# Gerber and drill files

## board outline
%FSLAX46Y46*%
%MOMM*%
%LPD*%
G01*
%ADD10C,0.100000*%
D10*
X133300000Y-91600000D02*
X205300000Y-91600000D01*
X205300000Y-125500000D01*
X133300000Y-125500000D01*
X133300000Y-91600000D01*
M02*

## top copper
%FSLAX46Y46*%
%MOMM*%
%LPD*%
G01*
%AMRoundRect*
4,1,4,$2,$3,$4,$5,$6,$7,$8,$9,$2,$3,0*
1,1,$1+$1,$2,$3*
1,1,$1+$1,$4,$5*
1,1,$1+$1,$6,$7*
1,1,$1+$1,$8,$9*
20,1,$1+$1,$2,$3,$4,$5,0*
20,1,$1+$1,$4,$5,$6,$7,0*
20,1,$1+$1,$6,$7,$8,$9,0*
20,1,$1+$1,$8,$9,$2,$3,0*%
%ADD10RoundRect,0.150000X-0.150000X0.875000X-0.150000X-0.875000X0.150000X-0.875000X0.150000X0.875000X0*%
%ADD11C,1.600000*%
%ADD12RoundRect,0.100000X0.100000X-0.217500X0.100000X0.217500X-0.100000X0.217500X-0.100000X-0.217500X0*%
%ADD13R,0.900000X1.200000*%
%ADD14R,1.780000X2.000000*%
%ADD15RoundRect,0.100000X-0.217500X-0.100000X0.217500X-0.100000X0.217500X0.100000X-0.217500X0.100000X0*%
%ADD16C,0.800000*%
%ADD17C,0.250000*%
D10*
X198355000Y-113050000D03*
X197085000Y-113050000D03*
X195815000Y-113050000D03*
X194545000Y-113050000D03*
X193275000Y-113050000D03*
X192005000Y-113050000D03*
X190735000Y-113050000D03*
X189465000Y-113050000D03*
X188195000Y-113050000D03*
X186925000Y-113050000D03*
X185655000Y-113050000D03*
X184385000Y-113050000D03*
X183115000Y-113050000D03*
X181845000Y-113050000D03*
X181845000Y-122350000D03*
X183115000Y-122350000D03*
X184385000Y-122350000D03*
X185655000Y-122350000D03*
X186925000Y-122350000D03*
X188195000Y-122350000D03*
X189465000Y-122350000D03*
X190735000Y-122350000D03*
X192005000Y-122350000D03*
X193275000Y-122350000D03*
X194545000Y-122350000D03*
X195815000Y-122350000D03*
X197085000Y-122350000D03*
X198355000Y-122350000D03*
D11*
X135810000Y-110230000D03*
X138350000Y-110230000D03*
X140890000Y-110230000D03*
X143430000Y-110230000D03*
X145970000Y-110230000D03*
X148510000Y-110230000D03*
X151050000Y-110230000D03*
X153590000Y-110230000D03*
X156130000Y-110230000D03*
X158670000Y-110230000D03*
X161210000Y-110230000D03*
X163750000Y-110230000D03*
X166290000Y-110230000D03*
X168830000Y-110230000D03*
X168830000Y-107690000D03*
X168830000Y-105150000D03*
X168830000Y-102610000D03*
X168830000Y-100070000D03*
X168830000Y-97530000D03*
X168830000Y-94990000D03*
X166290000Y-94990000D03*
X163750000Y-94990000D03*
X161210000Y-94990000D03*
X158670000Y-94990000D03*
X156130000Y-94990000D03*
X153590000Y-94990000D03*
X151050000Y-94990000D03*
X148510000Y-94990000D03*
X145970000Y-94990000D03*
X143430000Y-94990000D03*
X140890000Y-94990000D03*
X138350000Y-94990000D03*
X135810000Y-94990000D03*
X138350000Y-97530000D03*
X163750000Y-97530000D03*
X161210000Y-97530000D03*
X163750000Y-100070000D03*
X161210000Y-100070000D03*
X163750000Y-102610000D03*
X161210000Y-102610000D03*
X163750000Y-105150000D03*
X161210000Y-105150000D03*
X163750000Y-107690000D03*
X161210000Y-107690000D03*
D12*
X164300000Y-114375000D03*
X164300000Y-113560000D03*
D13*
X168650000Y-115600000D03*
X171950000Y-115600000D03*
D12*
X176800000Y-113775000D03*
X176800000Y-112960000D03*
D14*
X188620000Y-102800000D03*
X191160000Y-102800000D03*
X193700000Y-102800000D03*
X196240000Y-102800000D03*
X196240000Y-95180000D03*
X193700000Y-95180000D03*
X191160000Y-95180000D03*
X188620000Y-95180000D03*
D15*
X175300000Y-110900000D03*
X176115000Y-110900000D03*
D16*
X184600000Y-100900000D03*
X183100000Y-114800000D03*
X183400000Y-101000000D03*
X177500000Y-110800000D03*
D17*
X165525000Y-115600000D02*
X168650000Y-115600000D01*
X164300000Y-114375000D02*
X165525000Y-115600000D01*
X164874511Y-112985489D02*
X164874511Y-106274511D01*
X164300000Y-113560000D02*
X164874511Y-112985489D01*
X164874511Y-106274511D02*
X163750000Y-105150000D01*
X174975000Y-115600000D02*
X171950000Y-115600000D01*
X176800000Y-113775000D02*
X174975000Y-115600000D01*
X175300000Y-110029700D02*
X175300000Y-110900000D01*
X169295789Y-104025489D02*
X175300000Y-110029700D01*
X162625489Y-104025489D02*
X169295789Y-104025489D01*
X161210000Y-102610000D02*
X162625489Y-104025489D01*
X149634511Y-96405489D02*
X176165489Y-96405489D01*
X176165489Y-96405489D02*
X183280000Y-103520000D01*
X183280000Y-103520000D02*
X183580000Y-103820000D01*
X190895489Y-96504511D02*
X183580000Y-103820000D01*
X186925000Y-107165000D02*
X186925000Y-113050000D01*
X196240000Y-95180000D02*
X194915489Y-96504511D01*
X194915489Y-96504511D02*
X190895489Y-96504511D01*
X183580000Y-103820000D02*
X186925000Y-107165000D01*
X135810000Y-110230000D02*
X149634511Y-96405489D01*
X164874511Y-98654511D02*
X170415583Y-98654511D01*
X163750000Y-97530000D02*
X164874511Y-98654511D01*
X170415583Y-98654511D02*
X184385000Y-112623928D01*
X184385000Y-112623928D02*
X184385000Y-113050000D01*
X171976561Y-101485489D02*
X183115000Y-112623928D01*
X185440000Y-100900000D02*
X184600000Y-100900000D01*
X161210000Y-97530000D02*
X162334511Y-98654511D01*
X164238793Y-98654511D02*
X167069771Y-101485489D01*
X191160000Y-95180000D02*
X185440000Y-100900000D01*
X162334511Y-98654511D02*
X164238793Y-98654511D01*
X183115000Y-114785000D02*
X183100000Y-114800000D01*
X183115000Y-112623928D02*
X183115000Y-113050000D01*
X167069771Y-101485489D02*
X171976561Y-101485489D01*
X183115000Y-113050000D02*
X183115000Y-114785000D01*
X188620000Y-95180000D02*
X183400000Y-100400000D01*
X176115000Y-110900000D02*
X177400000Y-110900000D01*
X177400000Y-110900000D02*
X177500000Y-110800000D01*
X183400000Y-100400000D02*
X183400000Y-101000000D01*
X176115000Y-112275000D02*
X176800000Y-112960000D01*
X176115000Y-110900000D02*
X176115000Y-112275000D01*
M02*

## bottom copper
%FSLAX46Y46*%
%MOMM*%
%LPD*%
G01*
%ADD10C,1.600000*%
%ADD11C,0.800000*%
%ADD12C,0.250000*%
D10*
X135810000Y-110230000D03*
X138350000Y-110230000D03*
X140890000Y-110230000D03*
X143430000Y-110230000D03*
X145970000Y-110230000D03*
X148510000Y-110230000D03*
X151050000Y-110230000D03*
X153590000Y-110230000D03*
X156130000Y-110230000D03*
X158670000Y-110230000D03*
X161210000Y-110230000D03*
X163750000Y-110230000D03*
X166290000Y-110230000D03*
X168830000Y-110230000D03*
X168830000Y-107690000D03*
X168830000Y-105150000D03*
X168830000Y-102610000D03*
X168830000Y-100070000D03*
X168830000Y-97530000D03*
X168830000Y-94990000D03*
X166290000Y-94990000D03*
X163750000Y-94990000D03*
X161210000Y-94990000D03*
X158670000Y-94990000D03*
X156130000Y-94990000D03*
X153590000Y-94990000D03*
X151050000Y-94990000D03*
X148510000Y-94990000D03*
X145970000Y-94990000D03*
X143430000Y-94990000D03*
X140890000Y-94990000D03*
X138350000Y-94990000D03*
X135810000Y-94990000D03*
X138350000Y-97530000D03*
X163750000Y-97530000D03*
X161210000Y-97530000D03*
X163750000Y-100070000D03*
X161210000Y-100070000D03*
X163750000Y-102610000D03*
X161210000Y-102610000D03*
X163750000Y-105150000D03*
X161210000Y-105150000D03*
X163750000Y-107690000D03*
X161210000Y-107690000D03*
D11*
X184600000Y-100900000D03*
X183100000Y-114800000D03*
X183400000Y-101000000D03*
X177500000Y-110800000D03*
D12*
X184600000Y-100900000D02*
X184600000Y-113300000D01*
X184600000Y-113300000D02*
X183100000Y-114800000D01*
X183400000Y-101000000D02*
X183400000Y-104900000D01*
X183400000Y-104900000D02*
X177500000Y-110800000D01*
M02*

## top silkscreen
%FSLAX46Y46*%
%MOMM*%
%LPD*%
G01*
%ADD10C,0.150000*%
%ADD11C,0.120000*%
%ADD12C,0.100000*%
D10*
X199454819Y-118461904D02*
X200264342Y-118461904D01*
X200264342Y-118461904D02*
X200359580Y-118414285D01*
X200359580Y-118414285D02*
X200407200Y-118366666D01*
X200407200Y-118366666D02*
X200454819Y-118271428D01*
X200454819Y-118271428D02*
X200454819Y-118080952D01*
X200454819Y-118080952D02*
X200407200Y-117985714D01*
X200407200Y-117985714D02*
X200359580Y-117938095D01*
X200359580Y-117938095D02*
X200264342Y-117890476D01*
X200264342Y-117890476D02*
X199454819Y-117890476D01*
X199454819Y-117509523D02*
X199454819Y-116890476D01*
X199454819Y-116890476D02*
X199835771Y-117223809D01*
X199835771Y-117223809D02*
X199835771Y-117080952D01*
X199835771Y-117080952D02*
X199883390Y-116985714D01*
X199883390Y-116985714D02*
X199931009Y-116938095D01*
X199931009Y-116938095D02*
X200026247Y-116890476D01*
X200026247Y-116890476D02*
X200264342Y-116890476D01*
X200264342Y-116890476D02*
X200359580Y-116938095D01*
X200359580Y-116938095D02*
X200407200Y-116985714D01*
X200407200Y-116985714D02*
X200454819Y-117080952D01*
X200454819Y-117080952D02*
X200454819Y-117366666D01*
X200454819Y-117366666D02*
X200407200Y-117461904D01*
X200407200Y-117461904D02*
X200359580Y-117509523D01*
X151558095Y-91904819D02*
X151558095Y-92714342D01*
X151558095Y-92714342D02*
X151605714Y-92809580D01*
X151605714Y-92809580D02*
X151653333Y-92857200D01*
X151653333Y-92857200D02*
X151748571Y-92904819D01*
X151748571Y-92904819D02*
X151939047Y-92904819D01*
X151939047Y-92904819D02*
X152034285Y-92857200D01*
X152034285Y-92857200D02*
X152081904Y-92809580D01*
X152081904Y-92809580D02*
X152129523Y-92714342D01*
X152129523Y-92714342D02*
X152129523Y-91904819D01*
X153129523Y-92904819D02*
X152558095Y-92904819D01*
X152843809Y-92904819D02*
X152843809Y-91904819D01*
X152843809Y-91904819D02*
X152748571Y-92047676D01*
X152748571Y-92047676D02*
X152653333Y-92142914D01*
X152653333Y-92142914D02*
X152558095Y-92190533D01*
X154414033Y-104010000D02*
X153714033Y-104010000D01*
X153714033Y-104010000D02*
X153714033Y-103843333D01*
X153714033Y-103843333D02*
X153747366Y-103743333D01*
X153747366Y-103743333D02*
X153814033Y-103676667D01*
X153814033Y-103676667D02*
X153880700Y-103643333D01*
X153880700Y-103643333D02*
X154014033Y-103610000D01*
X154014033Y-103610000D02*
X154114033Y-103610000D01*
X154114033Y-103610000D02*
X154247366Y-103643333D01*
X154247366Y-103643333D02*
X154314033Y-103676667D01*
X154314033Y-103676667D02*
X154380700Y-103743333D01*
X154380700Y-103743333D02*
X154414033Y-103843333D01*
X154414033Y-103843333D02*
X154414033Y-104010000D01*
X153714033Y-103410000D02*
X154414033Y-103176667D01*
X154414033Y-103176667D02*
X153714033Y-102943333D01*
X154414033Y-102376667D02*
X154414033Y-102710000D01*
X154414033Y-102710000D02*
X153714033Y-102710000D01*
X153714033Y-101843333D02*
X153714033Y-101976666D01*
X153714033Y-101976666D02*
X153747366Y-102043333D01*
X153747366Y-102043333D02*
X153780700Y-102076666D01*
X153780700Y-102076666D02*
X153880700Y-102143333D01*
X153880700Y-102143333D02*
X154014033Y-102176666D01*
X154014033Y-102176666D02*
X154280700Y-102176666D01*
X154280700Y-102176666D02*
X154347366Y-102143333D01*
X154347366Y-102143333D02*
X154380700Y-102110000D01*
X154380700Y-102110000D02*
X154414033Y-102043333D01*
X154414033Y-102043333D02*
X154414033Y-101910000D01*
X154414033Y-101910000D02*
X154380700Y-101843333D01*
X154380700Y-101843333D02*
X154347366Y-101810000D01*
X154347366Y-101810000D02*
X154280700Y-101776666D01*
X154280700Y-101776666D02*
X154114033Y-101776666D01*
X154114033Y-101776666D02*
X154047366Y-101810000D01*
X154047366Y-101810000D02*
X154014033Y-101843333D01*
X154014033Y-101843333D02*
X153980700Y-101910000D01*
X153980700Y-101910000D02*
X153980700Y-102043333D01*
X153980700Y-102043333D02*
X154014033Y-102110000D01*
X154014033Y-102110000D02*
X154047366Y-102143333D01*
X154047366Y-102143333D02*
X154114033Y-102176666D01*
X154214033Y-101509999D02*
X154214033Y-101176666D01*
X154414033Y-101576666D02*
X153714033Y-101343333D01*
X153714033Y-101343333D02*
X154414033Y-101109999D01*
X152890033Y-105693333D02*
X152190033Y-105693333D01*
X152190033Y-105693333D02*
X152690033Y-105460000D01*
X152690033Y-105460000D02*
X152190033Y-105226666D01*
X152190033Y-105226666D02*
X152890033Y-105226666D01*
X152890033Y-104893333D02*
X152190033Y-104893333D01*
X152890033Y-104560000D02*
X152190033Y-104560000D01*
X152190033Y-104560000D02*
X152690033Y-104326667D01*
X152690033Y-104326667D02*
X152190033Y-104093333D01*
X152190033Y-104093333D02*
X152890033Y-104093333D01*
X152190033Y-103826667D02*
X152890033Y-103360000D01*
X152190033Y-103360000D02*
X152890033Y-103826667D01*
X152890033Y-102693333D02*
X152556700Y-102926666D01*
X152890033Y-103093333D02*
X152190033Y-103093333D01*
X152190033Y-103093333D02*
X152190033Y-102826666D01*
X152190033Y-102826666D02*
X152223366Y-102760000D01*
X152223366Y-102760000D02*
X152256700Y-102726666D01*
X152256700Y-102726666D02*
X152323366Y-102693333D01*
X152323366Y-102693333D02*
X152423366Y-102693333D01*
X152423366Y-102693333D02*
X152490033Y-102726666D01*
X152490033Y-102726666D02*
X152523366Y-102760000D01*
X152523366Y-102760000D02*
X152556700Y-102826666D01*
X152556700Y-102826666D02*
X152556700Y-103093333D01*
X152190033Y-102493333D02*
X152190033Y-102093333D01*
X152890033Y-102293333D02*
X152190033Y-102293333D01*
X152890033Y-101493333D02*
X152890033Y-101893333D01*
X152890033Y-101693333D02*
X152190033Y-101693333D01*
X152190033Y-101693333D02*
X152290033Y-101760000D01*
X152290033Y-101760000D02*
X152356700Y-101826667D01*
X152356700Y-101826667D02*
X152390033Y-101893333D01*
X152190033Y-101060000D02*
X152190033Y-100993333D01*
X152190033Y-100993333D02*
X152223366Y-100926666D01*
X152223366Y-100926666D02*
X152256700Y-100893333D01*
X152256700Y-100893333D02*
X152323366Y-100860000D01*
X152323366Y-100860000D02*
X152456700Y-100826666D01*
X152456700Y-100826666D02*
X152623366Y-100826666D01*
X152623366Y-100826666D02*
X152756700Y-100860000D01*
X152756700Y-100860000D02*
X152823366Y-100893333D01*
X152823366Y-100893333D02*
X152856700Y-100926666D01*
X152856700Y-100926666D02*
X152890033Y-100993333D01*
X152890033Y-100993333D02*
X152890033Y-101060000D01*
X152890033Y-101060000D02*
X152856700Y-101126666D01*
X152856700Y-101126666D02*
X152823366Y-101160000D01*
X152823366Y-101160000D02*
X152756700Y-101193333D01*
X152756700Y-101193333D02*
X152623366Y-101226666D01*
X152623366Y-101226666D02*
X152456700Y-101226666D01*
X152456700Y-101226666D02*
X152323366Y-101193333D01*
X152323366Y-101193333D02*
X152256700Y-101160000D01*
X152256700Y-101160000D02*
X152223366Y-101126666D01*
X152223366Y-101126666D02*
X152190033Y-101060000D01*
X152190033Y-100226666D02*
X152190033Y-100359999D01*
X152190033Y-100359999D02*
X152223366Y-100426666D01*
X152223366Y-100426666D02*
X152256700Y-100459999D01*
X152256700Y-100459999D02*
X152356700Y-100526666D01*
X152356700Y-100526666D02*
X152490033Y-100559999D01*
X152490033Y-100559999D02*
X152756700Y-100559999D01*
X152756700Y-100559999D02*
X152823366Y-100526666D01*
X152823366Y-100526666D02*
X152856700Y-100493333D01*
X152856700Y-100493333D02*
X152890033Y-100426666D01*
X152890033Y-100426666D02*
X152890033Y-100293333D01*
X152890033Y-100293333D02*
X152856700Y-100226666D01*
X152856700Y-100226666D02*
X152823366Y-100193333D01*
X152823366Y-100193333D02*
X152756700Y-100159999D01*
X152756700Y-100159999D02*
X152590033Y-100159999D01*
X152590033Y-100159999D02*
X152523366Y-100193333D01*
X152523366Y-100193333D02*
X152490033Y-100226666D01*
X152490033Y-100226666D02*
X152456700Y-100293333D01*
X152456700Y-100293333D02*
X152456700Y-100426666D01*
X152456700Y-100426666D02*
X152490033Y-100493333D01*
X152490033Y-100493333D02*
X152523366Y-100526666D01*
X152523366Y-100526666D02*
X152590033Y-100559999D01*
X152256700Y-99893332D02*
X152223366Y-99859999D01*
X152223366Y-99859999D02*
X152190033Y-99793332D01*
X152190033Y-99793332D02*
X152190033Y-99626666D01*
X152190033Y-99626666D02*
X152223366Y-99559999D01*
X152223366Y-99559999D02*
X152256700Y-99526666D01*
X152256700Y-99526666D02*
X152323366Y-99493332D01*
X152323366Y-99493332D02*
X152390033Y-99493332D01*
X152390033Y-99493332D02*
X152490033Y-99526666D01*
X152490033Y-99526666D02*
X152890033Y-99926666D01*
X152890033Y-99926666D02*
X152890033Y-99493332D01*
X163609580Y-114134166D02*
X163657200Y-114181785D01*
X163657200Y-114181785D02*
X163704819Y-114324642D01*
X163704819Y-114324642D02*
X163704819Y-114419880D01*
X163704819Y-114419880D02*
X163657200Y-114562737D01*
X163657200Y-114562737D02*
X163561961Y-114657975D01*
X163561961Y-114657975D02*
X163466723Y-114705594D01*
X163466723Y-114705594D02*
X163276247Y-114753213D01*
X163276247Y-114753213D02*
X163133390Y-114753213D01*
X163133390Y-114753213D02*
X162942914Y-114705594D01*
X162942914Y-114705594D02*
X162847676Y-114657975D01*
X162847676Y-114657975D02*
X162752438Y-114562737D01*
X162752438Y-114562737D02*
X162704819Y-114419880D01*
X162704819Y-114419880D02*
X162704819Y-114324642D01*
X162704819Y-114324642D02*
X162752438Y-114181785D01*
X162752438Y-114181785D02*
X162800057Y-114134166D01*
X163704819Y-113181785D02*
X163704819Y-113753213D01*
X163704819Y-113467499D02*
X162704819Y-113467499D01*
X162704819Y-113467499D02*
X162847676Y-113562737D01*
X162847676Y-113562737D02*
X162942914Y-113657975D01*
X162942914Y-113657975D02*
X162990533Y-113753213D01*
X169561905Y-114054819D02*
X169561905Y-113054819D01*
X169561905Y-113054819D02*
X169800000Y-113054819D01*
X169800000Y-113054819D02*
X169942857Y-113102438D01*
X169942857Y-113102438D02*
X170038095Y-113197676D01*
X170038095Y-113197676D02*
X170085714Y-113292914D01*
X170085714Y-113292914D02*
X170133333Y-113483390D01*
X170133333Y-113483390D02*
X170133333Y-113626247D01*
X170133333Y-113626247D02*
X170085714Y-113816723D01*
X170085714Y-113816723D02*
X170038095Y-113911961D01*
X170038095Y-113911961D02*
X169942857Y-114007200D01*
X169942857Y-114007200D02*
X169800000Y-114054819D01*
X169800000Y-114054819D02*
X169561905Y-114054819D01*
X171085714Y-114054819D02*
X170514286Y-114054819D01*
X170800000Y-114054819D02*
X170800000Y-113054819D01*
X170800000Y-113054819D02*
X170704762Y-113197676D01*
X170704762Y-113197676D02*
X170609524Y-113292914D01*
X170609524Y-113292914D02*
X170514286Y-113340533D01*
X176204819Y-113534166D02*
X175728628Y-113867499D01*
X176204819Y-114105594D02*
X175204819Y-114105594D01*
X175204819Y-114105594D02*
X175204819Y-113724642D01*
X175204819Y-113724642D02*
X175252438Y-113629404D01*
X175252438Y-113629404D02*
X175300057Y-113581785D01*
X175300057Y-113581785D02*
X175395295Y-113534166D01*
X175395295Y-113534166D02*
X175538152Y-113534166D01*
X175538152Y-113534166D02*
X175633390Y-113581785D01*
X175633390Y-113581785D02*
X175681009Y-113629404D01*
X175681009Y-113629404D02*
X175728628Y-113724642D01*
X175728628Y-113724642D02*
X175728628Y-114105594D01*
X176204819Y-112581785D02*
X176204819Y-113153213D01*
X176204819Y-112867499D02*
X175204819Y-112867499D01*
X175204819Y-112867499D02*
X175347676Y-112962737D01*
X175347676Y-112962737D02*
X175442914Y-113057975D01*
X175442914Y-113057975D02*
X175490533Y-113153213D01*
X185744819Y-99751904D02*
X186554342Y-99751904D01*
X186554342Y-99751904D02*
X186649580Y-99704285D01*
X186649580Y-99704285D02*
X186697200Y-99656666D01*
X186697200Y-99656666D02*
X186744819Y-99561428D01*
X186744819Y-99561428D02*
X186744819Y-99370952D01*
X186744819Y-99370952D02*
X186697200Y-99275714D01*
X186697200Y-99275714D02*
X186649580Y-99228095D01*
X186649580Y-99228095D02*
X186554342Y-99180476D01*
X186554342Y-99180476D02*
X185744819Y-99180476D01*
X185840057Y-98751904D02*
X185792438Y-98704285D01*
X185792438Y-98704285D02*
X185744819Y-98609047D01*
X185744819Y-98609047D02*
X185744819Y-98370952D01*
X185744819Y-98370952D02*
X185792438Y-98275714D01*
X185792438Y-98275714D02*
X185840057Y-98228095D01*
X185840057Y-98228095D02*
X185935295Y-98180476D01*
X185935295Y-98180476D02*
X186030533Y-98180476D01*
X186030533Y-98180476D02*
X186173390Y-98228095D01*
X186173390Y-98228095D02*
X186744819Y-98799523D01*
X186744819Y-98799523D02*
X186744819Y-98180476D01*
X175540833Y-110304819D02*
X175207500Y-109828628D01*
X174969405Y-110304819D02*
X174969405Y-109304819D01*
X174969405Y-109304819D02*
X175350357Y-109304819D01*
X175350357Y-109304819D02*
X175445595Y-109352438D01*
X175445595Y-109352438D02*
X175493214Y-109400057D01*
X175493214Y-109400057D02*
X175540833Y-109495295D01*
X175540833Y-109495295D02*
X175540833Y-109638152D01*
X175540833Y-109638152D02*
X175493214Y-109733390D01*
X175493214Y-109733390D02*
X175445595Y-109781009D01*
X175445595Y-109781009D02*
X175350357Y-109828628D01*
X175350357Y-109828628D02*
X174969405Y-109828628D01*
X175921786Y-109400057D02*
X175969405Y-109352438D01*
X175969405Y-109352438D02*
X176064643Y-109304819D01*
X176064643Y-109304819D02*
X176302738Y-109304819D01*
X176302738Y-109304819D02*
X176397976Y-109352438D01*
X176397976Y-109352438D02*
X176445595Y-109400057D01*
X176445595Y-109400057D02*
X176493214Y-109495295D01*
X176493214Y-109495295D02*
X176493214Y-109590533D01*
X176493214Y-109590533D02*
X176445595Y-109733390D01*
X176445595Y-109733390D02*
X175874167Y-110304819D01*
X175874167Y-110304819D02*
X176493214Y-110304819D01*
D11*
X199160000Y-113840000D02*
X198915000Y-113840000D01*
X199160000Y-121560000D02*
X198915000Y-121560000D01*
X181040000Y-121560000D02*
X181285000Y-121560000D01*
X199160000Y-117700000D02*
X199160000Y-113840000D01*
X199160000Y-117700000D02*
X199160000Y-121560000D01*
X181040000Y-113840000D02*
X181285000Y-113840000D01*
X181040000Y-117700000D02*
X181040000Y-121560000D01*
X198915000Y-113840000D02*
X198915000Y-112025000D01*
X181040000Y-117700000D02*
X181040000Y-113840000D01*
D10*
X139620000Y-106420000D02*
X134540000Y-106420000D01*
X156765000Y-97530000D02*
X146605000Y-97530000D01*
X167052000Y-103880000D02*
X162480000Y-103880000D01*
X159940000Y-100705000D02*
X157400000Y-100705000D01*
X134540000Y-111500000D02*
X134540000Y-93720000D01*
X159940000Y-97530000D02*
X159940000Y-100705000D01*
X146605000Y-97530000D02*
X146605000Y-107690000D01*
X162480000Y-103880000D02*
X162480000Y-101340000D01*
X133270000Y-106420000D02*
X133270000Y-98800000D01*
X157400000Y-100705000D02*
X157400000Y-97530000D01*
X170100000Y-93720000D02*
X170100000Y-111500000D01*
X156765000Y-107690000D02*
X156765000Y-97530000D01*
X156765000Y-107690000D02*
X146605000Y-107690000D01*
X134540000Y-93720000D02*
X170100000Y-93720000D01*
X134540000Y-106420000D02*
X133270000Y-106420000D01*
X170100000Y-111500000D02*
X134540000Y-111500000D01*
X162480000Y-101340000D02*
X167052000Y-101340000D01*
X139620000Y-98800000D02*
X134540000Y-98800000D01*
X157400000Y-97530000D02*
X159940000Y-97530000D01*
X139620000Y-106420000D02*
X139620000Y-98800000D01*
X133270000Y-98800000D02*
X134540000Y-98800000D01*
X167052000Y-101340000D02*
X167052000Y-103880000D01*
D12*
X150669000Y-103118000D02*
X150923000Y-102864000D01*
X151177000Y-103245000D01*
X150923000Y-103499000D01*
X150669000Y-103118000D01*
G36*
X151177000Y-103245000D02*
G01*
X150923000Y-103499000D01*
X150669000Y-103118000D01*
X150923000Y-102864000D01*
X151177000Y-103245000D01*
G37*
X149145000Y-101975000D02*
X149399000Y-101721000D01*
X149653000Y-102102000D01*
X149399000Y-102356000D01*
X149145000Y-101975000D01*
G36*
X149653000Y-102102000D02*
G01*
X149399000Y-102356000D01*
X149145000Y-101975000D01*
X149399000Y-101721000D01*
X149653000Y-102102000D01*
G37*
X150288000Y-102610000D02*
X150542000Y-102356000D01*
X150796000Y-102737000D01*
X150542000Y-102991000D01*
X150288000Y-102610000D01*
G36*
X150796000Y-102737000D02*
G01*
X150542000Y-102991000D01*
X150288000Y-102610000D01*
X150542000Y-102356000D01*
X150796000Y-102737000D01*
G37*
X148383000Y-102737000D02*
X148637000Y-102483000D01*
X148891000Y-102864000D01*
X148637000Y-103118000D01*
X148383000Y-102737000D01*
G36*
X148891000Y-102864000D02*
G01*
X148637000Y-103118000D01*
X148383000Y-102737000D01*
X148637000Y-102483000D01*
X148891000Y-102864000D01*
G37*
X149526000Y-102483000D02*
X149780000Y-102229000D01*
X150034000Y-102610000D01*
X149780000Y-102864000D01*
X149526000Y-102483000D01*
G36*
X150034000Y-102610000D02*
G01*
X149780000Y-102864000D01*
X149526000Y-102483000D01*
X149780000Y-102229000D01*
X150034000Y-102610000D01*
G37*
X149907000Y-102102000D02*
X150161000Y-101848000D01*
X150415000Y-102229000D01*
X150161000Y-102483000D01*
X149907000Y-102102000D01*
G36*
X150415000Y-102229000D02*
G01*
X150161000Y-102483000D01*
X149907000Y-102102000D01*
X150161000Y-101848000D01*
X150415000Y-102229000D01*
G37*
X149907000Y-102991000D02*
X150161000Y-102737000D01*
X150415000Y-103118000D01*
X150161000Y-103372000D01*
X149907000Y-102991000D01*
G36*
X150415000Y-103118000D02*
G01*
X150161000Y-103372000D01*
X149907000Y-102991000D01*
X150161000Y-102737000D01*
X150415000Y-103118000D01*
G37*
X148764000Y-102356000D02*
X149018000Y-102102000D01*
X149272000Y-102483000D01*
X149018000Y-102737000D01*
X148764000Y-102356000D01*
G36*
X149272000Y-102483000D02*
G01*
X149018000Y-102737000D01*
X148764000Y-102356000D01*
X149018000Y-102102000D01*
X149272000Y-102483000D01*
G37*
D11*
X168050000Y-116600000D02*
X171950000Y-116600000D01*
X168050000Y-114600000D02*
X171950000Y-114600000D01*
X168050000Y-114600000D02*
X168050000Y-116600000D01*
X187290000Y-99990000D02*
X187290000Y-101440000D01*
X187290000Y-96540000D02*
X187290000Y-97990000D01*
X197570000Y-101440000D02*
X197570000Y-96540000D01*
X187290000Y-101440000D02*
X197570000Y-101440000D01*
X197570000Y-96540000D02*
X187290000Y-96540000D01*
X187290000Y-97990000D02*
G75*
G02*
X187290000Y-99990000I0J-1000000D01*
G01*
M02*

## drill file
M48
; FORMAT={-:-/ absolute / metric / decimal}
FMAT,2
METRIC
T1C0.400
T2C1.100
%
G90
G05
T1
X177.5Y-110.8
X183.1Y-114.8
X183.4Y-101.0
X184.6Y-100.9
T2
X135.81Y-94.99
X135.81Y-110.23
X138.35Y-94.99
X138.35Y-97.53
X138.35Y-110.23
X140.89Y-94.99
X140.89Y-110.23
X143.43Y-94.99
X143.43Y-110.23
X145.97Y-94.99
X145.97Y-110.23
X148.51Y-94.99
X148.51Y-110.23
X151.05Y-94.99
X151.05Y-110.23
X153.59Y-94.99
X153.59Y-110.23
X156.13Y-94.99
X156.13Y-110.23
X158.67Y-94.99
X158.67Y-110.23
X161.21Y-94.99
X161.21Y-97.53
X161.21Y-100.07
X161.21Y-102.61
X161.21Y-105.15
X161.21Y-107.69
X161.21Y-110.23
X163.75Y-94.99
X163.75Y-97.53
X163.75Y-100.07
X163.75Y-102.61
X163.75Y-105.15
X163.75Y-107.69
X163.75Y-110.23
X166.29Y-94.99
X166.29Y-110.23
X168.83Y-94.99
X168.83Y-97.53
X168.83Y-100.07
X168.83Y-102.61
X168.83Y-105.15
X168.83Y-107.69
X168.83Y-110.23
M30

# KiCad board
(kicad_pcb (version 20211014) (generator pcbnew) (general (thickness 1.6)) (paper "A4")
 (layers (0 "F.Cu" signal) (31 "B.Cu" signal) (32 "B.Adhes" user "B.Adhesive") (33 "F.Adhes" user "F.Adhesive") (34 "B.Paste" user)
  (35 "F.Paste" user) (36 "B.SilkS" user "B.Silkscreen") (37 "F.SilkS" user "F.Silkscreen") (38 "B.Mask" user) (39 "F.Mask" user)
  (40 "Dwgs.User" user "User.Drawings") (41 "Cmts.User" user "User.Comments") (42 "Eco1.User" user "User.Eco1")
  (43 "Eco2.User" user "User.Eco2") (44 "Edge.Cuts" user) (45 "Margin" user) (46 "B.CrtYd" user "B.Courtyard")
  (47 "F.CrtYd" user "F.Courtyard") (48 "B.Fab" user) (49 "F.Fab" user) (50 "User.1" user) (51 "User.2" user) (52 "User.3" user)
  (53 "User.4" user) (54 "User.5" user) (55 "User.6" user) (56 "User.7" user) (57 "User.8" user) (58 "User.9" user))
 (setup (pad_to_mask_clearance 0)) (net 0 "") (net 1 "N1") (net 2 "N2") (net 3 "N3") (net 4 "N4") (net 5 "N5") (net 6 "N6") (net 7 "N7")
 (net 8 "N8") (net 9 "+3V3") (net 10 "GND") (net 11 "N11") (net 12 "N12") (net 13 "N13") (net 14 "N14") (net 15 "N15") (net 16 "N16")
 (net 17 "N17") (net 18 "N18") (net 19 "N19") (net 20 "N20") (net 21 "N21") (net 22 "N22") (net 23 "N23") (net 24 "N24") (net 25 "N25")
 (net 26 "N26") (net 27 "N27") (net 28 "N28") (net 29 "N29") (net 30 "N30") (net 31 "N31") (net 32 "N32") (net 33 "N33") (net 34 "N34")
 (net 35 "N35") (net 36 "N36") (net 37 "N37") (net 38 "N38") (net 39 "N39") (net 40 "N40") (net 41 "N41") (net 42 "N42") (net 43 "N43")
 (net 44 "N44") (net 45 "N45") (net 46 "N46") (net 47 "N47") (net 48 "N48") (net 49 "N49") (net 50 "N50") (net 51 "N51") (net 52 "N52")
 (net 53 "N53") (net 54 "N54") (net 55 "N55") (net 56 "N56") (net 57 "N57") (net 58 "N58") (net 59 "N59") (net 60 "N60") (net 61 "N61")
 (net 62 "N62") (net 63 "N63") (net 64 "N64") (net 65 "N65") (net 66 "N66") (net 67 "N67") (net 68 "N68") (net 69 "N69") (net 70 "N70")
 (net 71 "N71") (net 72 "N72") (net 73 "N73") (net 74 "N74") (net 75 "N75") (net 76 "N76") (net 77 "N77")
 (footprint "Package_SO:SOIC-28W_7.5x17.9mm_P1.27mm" (layer "F.Cu") (at 190.1 117.7 -90)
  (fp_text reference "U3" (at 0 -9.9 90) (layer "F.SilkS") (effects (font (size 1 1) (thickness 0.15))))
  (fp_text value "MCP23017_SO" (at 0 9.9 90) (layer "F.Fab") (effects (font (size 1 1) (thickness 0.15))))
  (fp_line (start -3.86 -9.06) (end -3.86 -8.815) (layer "F.SilkS") (width 0.12))
  (fp_line (start 3.86 -9.06) (end 3.86 -8.815) (layer "F.SilkS") (width 0.12))
  (fp_line (start 3.86 9.06) (end 3.86 8.815) (layer "F.SilkS") (width 0.12))
  (fp_line (start 0 -9.06) (end -3.86 -9.06) (layer "F.SilkS") (width 0.12))
  (fp_line (start 0 -9.06) (end 3.86 -9.06) (layer "F.SilkS") (width 0.12))
  (fp_line (start -3.86 9.06) (end -3.86 8.815) (layer "F.SilkS") (width 0.12))
  (fp_line (start 0 9.06) (end 3.86 9.06) (layer "F.SilkS") (width 0.12))
  (fp_line (start -3.86 -8.815) (end -5.675 -8.815) (layer "F.SilkS") (width 0.12))
  (fp_line (start 0 9.06) (end -3.86 9.06) (layer "F.SilkS") (width 0.12))
  (pad "1" smd roundrect (at -4.65 -8.255 270) (size 2.05 0.6) (layers "F.Cu" "F.Paste" "F.Mask") (roundrect_rratio 0.25) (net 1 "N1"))
  (pad "2" smd roundrect (at -4.65 -6.985 270) (size 2.05 0.6) (layers "F.Cu" "F.Paste" "F.Mask") (roundrect_rratio 0.25) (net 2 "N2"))
  (pad "3" smd roundrect (at -4.65 -5.715 270) (size 2.05 0.6) (layers "F.Cu" "F.Paste" "F.Mask") (roundrect_rratio 0.25) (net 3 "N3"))
  (pad "4" smd roundrect (at -4.65 -4.445 270) (size 2.05 0.6) (layers "F.Cu" "F.Paste" "F.Mask") (roundrect_rratio 0.25) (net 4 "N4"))
  (pad "5" smd roundrect (at -4.65 -3.175 270) (size 2.05 0.6) (layers "F.Cu" "F.Paste" "F.Mask") (roundrect_rratio 0.25) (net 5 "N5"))
  (pad "6" smd roundrect (at -4.65 -1.905 270) (size 2.05 0.6) (layers "F.Cu" "F.Paste" "F.Mask") (roundrect_rratio 0.25) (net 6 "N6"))
  (pad "7" smd roundrect (at -4.65 -0.635 270) (size 2.05 0.6) (layers "F.Cu" "F.Paste" "F.Mask") (roundrect_rratio 0.25) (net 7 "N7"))
  (pad "8" smd roundrect (at -4.65 0.635 270) (size 2.05 0.6) (layers "F.Cu" "F.Paste" "F.Mask") (roundrect_rratio 0.25) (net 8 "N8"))
  (pad "9" smd roundrect (at -4.65 1.905 270) (size 2.05 0.6) (layers "F.Cu" "F.Paste" "F.Mask") (roundrect_rratio 0.25) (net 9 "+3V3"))
  (pad "10" smd roundrect (at -4.65 3.175 270) (size 2.05 0.6) (layers "F.Cu" "F.Paste" "F.Mask") (roundrect_rratio 0.25) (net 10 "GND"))
  (pad "11" smd roundrect (at -4.65 4.445 270) (size 2.05 0.6) (layers "F.Cu" "F.Paste" "F.Mask") (roundrect_rratio 0.25) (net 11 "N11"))
  (pad "12" smd roundrect (at -4.65 5.715 270) (size 2.05 0.6) (layers "F.Cu" "F.Paste" "F.Mask") (roundrect_rratio 0.25) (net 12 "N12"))
  (pad "13" smd roundrect (at -4.65 6.985 270) (size 2.05 0.6) (layers "F.Cu" "F.Paste" "F.Mask") (roundrect_rratio 0.25) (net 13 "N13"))
  (pad "14" smd roundrect (at -4.65 8.255 270) (size 2.05 0.6) (layers "F.Cu" "F.Paste" "F.Mask") (roundrect_rratio 0.25) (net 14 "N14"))
  (pad "15" smd roundrect (at 4.65 8.255 270) (size 2.05 0.6) (layers "F.Cu" "F.Paste" "F.Mask") (roundrect_rratio 0.25) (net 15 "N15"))
  (pad "16" smd roundrect (at 4.65 6.985 270) (size 2.05 0.6) (layers "F.Cu" "F.Paste" "F.Mask") (roundrect_rratio 0.25) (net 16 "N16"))
  (pad "17" smd roundrect (at 4.65 5.715 270) (size 2.05 0.6) (layers "F.Cu" "F.Paste" "F.Mask") (roundrect_rratio 0.25) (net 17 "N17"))
  (pad "18" smd roundrect (at 4.65 4.445 270) (size 2.05 0.6) (layers "F.Cu" "F.Paste" "F.Mask") (roundrect_rratio 0.25) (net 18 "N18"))
  (pad "19" smd roundrect (at 4.65 3.175 270) (size 2.05 0.6) (layers "F.Cu" "F.Paste" "F.Mask") (roundrect_rratio 0.25) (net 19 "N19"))
  (pad "20" smd roundrect (at 4.65 1.905 270) (size 2.05 0.6) (layers "F.Cu" "F.Paste" "F.Mask") (roundrect_rratio 0.25) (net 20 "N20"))
  (pad "21" smd roundrect (at 4.65 0.635 270) (size 2.05 0.6) (layers "F.Cu" "F.Paste" "F.Mask") (roundrect_rratio 0.25) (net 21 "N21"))
  (pad "22" smd roundrect (at 4.65 -0.635 270) (size 2.05 0.6) (layers "F.Cu" "F.Paste" "F.Mask") (roundrect_rratio 0.25) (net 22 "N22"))
  (pad "23" smd roundrect (at 4.65 -1.905 270) (size 2.05 0.6) (layers "F.Cu" "F.Paste" "F.Mask") (roundrect_rratio 0.25) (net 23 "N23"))
  (pad "24" smd roundrect (at 4.65 -3.175 270) (size 2.05 0.6) (layers "F.Cu" "F.Paste" "F.Mask") (roundrect_rratio 0.25) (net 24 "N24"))
  (pad "25" smd roundrect (at 4.65 -4.445 270) (size 2.05 0.6) (layers "F.Cu" "F.Paste" "F.Mask") (roundrect_rratio 0.25) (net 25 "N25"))
  (pad "26" smd roundrect (at 4.65 -5.715 270) (size 2.05 0.6) (layers "F.Cu" "F.Paste" "F.Mask") (roundrect_rratio 0.25) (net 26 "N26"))
  (pad "27" smd roundrect (at 4.65 -6.985 270) (size 2.05 0.6) (layers "F.Cu" "F.Paste" "F.Mask") (roundrect_rratio 0.25) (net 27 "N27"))
  (pad "28" smd roundrect (at 4.65 -8.255 270) (size 2.05 0.6) (layers "F.Cu" "F.Paste" "F.Mask") (roundrect_rratio 0.25) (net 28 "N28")))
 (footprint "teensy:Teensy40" (layer "F.Cu") (at 152.32 102.61)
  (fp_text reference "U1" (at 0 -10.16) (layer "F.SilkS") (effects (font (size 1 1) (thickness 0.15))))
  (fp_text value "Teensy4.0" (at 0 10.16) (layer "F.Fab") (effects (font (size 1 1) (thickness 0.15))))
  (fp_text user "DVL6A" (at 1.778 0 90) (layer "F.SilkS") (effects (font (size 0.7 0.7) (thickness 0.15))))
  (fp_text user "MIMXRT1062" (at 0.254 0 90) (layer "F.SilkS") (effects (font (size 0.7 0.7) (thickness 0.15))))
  (fp_line (start -12.7 3.81) (end -17.78 3.81) (layer "F.SilkS") (width 0.15))
  (fp_line (start 4.445 -5.08) (end -5.715 -5.08) (layer "F.SilkS") (width 0.15))
  (fp_line (start 14.732 1.27) (end 10.16 1.27) (layer "F.SilkS") (width 0.15))
  (fp_line (start 7.62 -1.905) (end 5.08 -1.905) (layer "F.SilkS") (width 0.15))
  (fp_line (start -17.78 8.89) (end -17.78 -8.89) (layer "F.SilkS") (width 0.15))
  (fp_line (start 7.62 -5.08) (end 7.62 -1.905) (layer "F.SilkS") (width 0.15))
  (fp_line (start -5.715 -5.08) (end -5.715 5.08) (layer "F.SilkS") (width 0.15))
  (fp_line (start 10.16 1.27) (end 10.16 -1.27) (layer "F.SilkS") (width 0.15))
  (fp_line (start -19.05 3.81) (end -19.05 -3.81) (layer "F.SilkS") (width 0.15))
  (fp_line (start 5.08 -1.905) (end 5.08 -5.08) (layer "F.SilkS") (width 0.15))
  (fp_line (start 17.78 -8.89) (end 17.78 8.89) (layer "F.SilkS") (width 0.15))
  (fp_line (start 4.445 5.08) (end 4.445 -5.08) (layer "F.SilkS") (width 0.15))
  (fp_line (start 4.445 5.08) (end -5.715 5.08) (layer "F.SilkS") (width 0.15))
  (fp_line (start -17.78 -8.89) (end 17.78 -8.89) (layer "F.SilkS") (width 0.15))
  (fp_line (start -17.78 3.81) (end -19.05 3.81) (layer "F.SilkS") (width 0.15))
  (fp_line (start 17.78 8.89) (end -17.78 8.89) (layer "F.SilkS") (width 0.15))
  (fp_line (start 10.16 -1.27) (end 14.732 -1.27) (layer "F.SilkS") (width 0.15))
  (fp_line (start -12.7 -3.81) (end -17.78 -3.81) (layer "F.SilkS") (width 0.15))
  (fp_line (start 5.08 -5.08) (end 7.62 -5.08) (layer "F.SilkS") (width 0.15))
  (fp_line (start -12.7 3.81) (end -12.7 -3.81) (layer "F.SilkS") (width 0.15))
  (fp_line (start -19.05 -3.81) (end -17.78 -3.81) (layer "F.SilkS") (width 0.15))
  (fp_line (start 14.732 -1.27) (end 14.732 1.27) (layer "F.SilkS") (width 0.15))
  (fp_poly (pts (xy -1.651 0.508) (xy -1.397 0.254) (xy -1.143 0.635) (xy -1.397 0.889)) (layer "F.SilkS") (width 0.1) (fill solid))
  (fp_poly (pts (xy -3.175 -0.635) (xy -2.921 -0.889) (xy -2.667 -0.508) (xy -2.921 -0.254)) (layer "F.SilkS") (width 0.1) (fill solid))
  (fp_poly (pts (xy -2.032 0) (xy -1.778 -0.254) (xy -1.524 0.127) (xy -1.778 0.381)) (layer "F.SilkS") (width 0.1) (fill solid))
  (fp_poly (pts (xy -3.937 0.127) (xy -3.683 -0.127) (xy -3.429 0.254) (xy -3.683 0.508)) (layer "F.SilkS") (width 0.1) (fill solid))
  (fp_poly (pts (xy -2.794 -0.127) (xy -2.54 -0.381) (xy -2.286 0) (xy -2.54 0.254)) (layer "F.SilkS") (width 0.1) (fill solid))
  (fp_poly (pts (xy -2.413 -0.508) (xy -2.159 -0.762) (xy -1.905 -0.381) (xy -2.159 -0.127)) (layer "F.SilkS") (width 0.1) (fill solid))
  (fp_poly (pts (xy -2.413 0.381) (xy -2.159 0.127) (xy -1.905 0.508) (xy -2.159 0.762)) (layer "F.SilkS") (width 0.1) (fill solid))
  (fp_poly (pts (xy -3.556 -0.254) (xy -3.302 -0.508) (xy -3.048 -0.127) (xy -3.302 0.127)) (layer "F.SilkS") (width 0.1) (fill solid))
  (pad "1" thru_hole circle locked (at -16.51 7.62) (size 1.6 1.6) (drill 1.1) (layers *.Cu *.Mask) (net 10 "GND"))
  (pad "2" thru_hole circle locked (at -13.97 7.62) (size 1.6 1.6) (drill 1.1) (layers *.Cu *.Mask) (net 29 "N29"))
  (pad "3" thru_hole circle locked (at -11.43 7.62) (size 1.6 1.6) (drill 1.1) (layers *.Cu *.Mask) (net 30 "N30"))
  (pad "4" thru_hole circle locked (at -8.89 7.62) (size 1.6 1.6) (drill 1.1) (layers *.Cu *.Mask) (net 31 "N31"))
  (pad "5" thru_hole circle locked (at -6.35 7.62) (size 1.6 1.6) (drill 1.1) (layers *.Cu *.Mask) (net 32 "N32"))
  (pad "6" thru_hole circle locked (at -3.81 7.62) (size 1.6 1.6) (drill 1.1) (layers *.Cu *.Mask) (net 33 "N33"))
  (pad "7" thru_hole circle locked (at -1.27 7.62) (size 1.6 1.6) (drill 1.1) (layers *.Cu *.Mask) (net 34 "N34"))
  (pad "8" thru_hole circle locked (at 1.27 7.62) (size 1.6 1.6) (drill 1.1) (layers *.Cu *.Mask) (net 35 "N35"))
  (pad "9" thru_hole circle locked (at 3.81 7.62) (size 1.6 1.6) (drill 1.1) (layers *.Cu *.Mask) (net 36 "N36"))
  (pad "10" thru_hole circle locked (at 6.35 7.62) (size 1.6 1.6) (drill 1.1) (layers *.Cu *.Mask) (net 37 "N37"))
  (pad "11" thru_hole circle locked (at 8.89 7.62) (size 1.6 1.6) (drill 1.1) (layers *.Cu *.Mask) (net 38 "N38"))
  (pad "12" thru_hole circle locked (at 11.43 7.62) (size 1.6 1.6) (drill 1.1) (layers *.Cu *.Mask) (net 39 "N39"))
  (pad "13" thru_hole circle locked (at 13.97 7.62) (size 1.6 1.6) (drill 1.1) (layers *.Cu *.Mask) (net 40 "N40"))
  (pad "14" thru_hole circle locked (at 16.51 7.62) (size 1.6 1.6) (drill 1.1) (layers *.Cu *.Mask) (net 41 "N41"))
  (pad "15" thru_hole circle locked (at 16.51 5.08) (size 1.6 1.6) (drill 1.1) (layers *.Cu *.Mask) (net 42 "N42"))
  (pad "16" thru_hole circle locked (at 16.51 2.54) (size 1.6 1.6) (drill 1.1) (layers *.Cu *.Mask) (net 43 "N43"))
  (pad "17" thru_hole circle locked (at 16.51 0) (size 1.6 1.6) (drill 1.1) (layers *.Cu *.Mask) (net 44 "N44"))
  (pad "18" thru_hole circle locked (at 16.51 -2.54) (size 1.6 1.6) (drill 1.1) (layers *.Cu *.Mask) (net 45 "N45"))
  (pad "19" thru_hole circle locked (at 16.51 -5.08) (size 1.6 1.6) (drill 1.1) (layers *.Cu *.Mask) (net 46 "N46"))
  (pad "20" thru_hole circle locked (at 16.51 -7.62) (size 1.6 1.6) (drill 1.1) (layers *.Cu *.Mask) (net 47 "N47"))
  (pad "21" thru_hole circle locked (at 13.97 -7.62) (size 1.6 1.6) (drill 1.1) (layers *.Cu *.Mask) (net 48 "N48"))
  (pad "22" thru_hole circle locked (at 11.43 -7.62) (size 1.6 1.6) (drill 1.1) (layers *.Cu *.Mask) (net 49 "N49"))
  (pad "23" thru_hole circle locked (at 8.89 -7.62) (size 1.6 1.6) (drill 1.1) (layers *.Cu *.Mask) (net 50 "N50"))
  (pad "24" thru_hole circle locked (at 6.35 -7.62) (size 1.6 1.6) (drill 1.1) (layers *.Cu *.Mask) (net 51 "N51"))
  (pad "25" thru_hole circle locked (at 3.81 -7.62) (size 1.6 1.6) (drill 1.1) (layers *.Cu *.Mask) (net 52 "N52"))
  (pad "26" thru_hole circle locked (at 1.27 -7.62) (size 1.6 1.6) (drill 1.1) (layers *.Cu *.Mask) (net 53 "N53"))
  (pad "27" thru_hole circle locked (at -1.27 -7.62) (size 1.6 1.6) (drill 1.1) (layers *.Cu *.Mask) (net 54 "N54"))
  (pad "28" thru_hole circle locked (at -3.81 -7.62) (size 1.6 1.6) (drill 1.1) (layers *.Cu *.Mask) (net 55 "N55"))
  (pad "29" thru_hole circle locked (at -6.35 -7.62) (size 1.6 1.6) (drill 1.1) (layers *.Cu *.Mask) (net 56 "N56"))
  (pad "30" thru_hole circle locked (at -8.89 -7.62) (size 1.6 1.6) (drill 1.1) (layers *.Cu *.Mask) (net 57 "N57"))
  (pad "31" thru_hole circle locked (at -11.43 -7.62) (size 1.6 1.6) (drill 1.1) (layers *.Cu *.Mask) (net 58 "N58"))
  (pad "32" thru_hole circle locked (at -13.97 -7.62) (size 1.6 1.6) (drill 1.1) (layers *.Cu *.Mask) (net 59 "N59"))
  (pad "33" thru_hole circle locked (at -16.51 -7.62) (size 1.6 1.6) (drill 1.1) (layers *.Cu *.Mask) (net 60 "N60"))
  (pad "34" thru_hole circle locked (at -13.97 -5.08) (size 1.6 1.6) (drill 1.1) (layers *.Cu *.Mask) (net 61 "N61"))
  (pad "35" thru_hole circle locked (at 11.43 -5.08) (size 1.6 1.6) (drill 1.1) (layers *.Cu *.Mask) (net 12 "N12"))
  (pad "36" thru_hole circle locked (at 8.89 -5.08) (size 1.6 1.6) (drill 1.1) (layers *.Cu *.Mask) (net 13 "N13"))
  (pad "37" thru_hole circle locked (at 11.43 -2.54) (size 1.6 1.6) (drill 1.1) (layers *.Cu *.Mask) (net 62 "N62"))
  (pad "38" thru_hole circle locked (at 8.89 -2.54) (size 1.6 1.6) (drill 1.1) (layers *.Cu *.Mask) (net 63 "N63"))
  (pad "39" thru_hole circle locked (at 11.43 0) (size 1.6 1.6) (drill 1.1) (layers *.Cu *.Mask) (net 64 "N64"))
  (pad "40" thru_hole circle locked (at 8.89 0) (size 1.6 1.6) (drill 1.1) (layers *.Cu *.Mask) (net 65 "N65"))
  (pad "41" thru_hole circle locked (at 11.43 2.54) (size 1.6 1.6) (drill 1.1) (layers *.Cu *.Mask) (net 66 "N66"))
  (pad "42" thru_hole circle locked (at 8.89 2.54) (size 1.6 1.6) (drill 1.1) (layers *.Cu *.Mask) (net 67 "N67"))
  (pad "43" thru_hole circle locked (at 11.43 5.08) (size 1.6 1.6) (drill 1.1) (layers *.Cu *.Mask) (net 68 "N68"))
  (pad "44" thru_hole circle locked (at 8.89 5.08) (size 1.6 1.6) (drill 1.1) (layers *.Cu *.Mask) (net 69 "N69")))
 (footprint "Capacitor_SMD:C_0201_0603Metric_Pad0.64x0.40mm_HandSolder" (layer "F.Cu") (at 164.3 113.9675 90)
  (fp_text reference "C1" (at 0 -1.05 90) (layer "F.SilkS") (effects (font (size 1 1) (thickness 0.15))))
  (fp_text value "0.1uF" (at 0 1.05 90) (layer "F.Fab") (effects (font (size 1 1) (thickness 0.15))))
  (pad "" smd roundrect (at -0.4325 0 90) (size 0.458 0.36) (layers "F.Paste") (roundrect_rratio 0.25))
  (pad "" smd roundrect (at 0.4325 0 90) (size 0.458 0.36) (layers "F.Paste") (roundrect_rratio 0.25))
  (pad "1" smd roundrect (at -0.4075 0 90) (size 0.635 0.4) (layers "F.Cu" "F.Mask") (roundrect_rratio 0.25) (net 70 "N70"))
  (pad "2" smd roundrect (at 0.4075 0 90) (size 0.635 0.4) (layers "F.Cu" "F.Mask") (roundrect_rratio 0.25) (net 66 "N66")))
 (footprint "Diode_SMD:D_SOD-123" (layer "F.Cu") (at 170.3 115.6)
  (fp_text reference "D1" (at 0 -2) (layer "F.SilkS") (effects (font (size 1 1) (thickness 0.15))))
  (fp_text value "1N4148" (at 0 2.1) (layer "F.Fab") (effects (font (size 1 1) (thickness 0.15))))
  (fp_line (start -2.25 1) (end 1.65 1) (layer "F.SilkS") (width 0.12))
  (fp_line (start -2.25 -1) (end 1.65 -1) (layer "F.SilkS") (width 0.12))
  (fp_line (start -2.25 -1) (end -2.25 1) (layer "F.SilkS") (width 0.12))
  (pad "1" smd rect (at -1.65 0) (size 0.9 1.2) (layers "F.Cu" "F.Paste" "F.Mask") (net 70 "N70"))
  (pad "2" smd rect (at 1.65 0) (size 0.9 1.2) (layers "F.Cu" "F.Paste" "F.Mask") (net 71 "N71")))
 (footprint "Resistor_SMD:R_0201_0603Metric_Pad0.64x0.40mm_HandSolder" (layer "F.Cu") (at 176.8 113.3675 90)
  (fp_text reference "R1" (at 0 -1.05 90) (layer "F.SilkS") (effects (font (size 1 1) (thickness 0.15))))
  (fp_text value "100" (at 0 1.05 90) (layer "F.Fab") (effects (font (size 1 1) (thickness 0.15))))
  (pad "" smd roundrect (at -0.4325 0 90) (size 0.458 0.36) (layers "F.Paste") (roundrect_rratio 0.25))
  (pad "" smd roundrect (at 0.4325 0 90) (size 0.458 0.36) (layers "F.Paste") (roundrect_rratio 0.25))
  (pad "1" smd roundrect (at -0.4075 0 90) (size 0.635 0.4) (layers "F.Cu" "F.Mask") (roundrect_rratio 0.25) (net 71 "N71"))
  (pad "2" smd roundrect (at 0.4075 0 90) (size 0.635 0.4) (layers "F.Cu" "F.Mask") (roundrect_rratio 0.25) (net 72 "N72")))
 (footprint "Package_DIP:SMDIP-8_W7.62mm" (layer "F.Cu") (at 192.43 98.99 90)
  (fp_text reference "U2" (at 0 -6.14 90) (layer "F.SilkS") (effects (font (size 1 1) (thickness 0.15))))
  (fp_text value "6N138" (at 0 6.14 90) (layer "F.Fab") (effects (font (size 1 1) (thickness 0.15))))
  (fp_line (start -1 -5.14) (end -2.45 -5.14) (layer "F.SilkS") (width 0.12))
  (fp_line (start 2.45 -5.14) (end 1 -5.14) (layer "F.SilkS") (width 0.12))
  (fp_line (start -2.45 5.14) (end 2.45 5.14) (layer "F.SilkS") (width 0.12))
  (fp_line (start -2.45 -5.14) (end -2.45 5.14) (layer "F.SilkS") (width 0.12))
  (fp_line (start 2.45 5.14) (end 2.45 -5.14) (layer "F.SilkS") (width 0.12))
  (fp_arc (start 1 -5.14) (mid 0 -4.14) (end -1 -5.14) (layer "F.SilkS") (width 0.12))
  (pad "1" smd rect (at -3.81 -3.81 90) (size 2 1.78) (layers "F.Cu" "F.Paste" "F.Mask") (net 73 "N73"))
  (pad "2" smd rect (at -3.81 -1.27 90) (size 2 1.78) (layers "F.Cu" "F.Paste" "F.Mask") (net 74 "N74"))
  (pad "3" smd rect (at -3.81 1.27 90) (size 2 1.78) (layers "F.Cu" "F.Paste" "F.Mask") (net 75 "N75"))
  (pad "4" smd rect (at -3.81 3.81 90) (size 2 1.78) (layers "F.Cu" "F.Paste" "F.Mask") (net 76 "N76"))
  (pad "5" smd rect (at 3.81 3.81 90) (size 2 1.78) (layers "F.Cu" "F.Paste" "F.Mask") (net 10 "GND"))
  (pad "6" smd rect (at 3.81 1.27 90) (size 2 1.78) (layers "F.Cu" "F.Paste" "F.Mask") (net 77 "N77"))
  (pad "7" smd rect (at 3.81 -1.27 90) (size 2 1.78) (layers "F.Cu" "F.Paste" "F.Mask") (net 13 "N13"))
  (pad "8" smd rect (at 3.81 -3.81 90) (size 2 1.78) (layers "F.Cu" "F.Paste" "F.Mask") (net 72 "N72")))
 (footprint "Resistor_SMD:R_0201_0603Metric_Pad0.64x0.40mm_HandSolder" (layer "F.Cu") (at 175.7075 110.9)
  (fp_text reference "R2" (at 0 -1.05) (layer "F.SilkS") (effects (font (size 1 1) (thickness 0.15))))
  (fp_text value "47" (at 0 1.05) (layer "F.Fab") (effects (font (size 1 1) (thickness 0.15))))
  (pad "" smd roundrect (at -0.4325 0) (size 0.458 0.36) (layers "F.Paste") (roundrect_rratio 0.25))
  (pad "" smd roundrect (at 0.4325 0) (size 0.458 0.36) (layers "F.Paste") (roundrect_rratio 0.25))
  (pad "1" smd roundrect (at -0.4075 0) (size 0.635 0.4) (layers "F.Cu" "F.Mask") (roundrect_rratio 0.25) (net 65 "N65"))
  (pad "2" smd roundrect (at 0.4075 0) (size 0.635 0.4) (layers "F.Cu" "F.Mask") (roundrect_rratio 0.25) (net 72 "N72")))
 (gr_rect (start 205.3 125.5) (end 133.3 91.6) (layer "Edge.Cuts") (width 0.1) (fill none))
 (segment (start 165.525 115.6) (end 168.65 115.6) (width 0.25) (layer "F.Cu") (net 70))
 (segment (start 164.3 114.375) (end 165.525 115.6) (width 0.25) (layer "F.Cu") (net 70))
 (segment (start 164.874511 112.985489) (end 164.874511 106.274511) (width 0.25) (layer "F.Cu") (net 66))
 (segment (start 164.3 113.56) (end 164.874511 112.985489) (width 0.25) (layer "F.Cu") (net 66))
 (segment (start 164.874511 106.274511) (end 163.75 105.15) (width 0.25) (layer "F.Cu") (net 66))
 (segment (start 174.975 115.6) (end 171.95 115.6) (width 0.25) (layer "F.Cu") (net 71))
 (segment (start 176.8 113.775) (end 174.975 115.6) (width 0.25) (layer "F.Cu") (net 71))
 (segment (start 175.3 110.0297) (end 175.3 110.9) (width 0.25) (layer "F.Cu") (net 65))
 (segment (start 169.295789 104.025489) (end 175.3 110.0297) (width 0.25) (layer "F.Cu") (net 65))
 (segment (start 162.625489 104.025489) (end 169.295789 104.025489) (width 0.25) (layer "F.Cu") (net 65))
 (segment (start 161.21 102.61) (end 162.625489 104.025489) (width 0.25) (layer "F.Cu") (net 65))
 (segment (start 149.634511 96.405489) (end 176.165489 96.405489) (width 0.25) (layer "F.Cu") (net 10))
 (segment (start 176.165489 96.405489) (end 183.28 103.52) (width 0.25) (layer "F.Cu") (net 10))
 (segment (start 183.28 103.52) (end 183.58 103.82) (width 0.25) (layer "F.Cu") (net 10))
 (segment (start 190.895489 96.504511) (end 183.58 103.82) (width 0.25) (layer "F.Cu") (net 10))
 (segment (start 186.925 107.165) (end 186.925 113.05) (width 0.25) (layer "F.Cu") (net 10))
 (segment (start 196.24 95.18) (end 194.915489 96.504511) (width 0.25) (layer "F.Cu") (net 10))
 (segment (start 194.915489 96.504511) (end 190.895489 96.504511) (width 0.25) (layer "F.Cu") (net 10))
 (segment (start 183.58 103.82) (end 186.925 107.165) (width 0.25) (layer "F.Cu") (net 10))
 (segment (start 135.81 110.23) (end 149.634511 96.405489) (width 0.25) (layer "F.Cu") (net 10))
 (segment (start 164.874511 98.654511) (end 170.415583 98.654511) (width 0.25) (layer "F.Cu") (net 12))
 (segment (start 163.75 97.53) (end 164.874511 98.654511) (width 0.25) (layer "F.Cu") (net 12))
 (segment (start 170.415583 98.654511) (end 184.385 112.623928) (width 0.25) (layer "F.Cu") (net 12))
 (segment (start 184.385 112.623928) (end 184.385 113.05) (width 0.25) (layer "F.Cu") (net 12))
 (segment (start 171.976561 101.485489) (end 183.115 112.623928) (width 0.25) (layer "F.Cu") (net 13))
 (segment (start 185.44 100.9) (end 184.6 100.9) (width 0.25) (layer "F.Cu") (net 13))
 (segment (start 161.21 97.53) (end 162.334511 98.654511) (width 0.25) (layer "F.Cu") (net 13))
 (segment (start 164.238793 98.654511) (end 167.069771 101.485489) (width 0.25) (layer "F.Cu") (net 13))
 (segment (start 191.16 95.18) (end 185.44 100.9) (width 0.25) (layer "F.Cu") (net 13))
 (segment (start 162.334511 98.654511) (end 164.238793 98.654511) (width 0.25) (layer "F.Cu") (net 13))
 (segment (start 183.115 114.785) (end 183.1 114.8) (width 0.25) (layer "F.Cu") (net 13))
 (segment (start 183.115 112.623928) (end 183.115 113.05) (width 0.25) (layer "F.Cu") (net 13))
 (segment (start 167.069771 101.485489) (end 171.976561 101.485489) (width 0.25) (layer "F.Cu") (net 13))
 (segment (start 183.115 113.05) (end 183.115 114.785) (width 0.25) (layer "F.Cu") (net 13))
 (via (at 184.6 100.9) (size 0.8) (drill 0.4) (layers "F.Cu" "B.Cu") (free) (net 13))
 (via (at 183.1 114.8) (size 0.8) (drill 0.4) (layers "F.Cu" "B.Cu") (free) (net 13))
 (segment (start 184.6 100.9) (end 184.6 113.3) (width 0.25) (layer "B.Cu") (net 13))
 (segment (start 184.6 113.3) (end 183.1 114.8) (width 0.25) (layer "B.Cu") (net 13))
 (segment (start 188.62 95.18) (end 183.4 100.4) (width 0.25) (layer "F.Cu") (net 72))
 (segment (start 176.115 110.9) (end 177.4 110.9) (width 0.25) (layer "F.Cu") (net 72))
 (segment (start 177.4 110.9) (end 177.5 110.8) (width 0.25) (layer "F.Cu") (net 72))
 (segment (start 183.4 100.4) (end 183.4 101) (width 0.25) (layer "F.Cu") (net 72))
 (segment (start 176.115 112.275) (end 176.8 112.96) (width 0.25) (layer "F.Cu") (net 72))
 (segment (start 176.115 110.9) (end 176.115 112.275) (width 0.25) (layer "F.Cu") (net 72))
 (via (at 183.4 101) (size 0.8) (drill 0.4) (layers "F.Cu" "B.Cu") (free) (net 72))
 (via (at 177.5 110.8) (size 0.8) (drill 0.4) (layers "F.Cu" "B.Cu") (free) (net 72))
 (segment (start 183.4 101) (end 183.4 104.9) (width 0.25) (layer "B.Cu") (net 72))
 (segment (start 183.4 104.9) (end 177.5 110.8) (width 0.25) (layer "B.Cu") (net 72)))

